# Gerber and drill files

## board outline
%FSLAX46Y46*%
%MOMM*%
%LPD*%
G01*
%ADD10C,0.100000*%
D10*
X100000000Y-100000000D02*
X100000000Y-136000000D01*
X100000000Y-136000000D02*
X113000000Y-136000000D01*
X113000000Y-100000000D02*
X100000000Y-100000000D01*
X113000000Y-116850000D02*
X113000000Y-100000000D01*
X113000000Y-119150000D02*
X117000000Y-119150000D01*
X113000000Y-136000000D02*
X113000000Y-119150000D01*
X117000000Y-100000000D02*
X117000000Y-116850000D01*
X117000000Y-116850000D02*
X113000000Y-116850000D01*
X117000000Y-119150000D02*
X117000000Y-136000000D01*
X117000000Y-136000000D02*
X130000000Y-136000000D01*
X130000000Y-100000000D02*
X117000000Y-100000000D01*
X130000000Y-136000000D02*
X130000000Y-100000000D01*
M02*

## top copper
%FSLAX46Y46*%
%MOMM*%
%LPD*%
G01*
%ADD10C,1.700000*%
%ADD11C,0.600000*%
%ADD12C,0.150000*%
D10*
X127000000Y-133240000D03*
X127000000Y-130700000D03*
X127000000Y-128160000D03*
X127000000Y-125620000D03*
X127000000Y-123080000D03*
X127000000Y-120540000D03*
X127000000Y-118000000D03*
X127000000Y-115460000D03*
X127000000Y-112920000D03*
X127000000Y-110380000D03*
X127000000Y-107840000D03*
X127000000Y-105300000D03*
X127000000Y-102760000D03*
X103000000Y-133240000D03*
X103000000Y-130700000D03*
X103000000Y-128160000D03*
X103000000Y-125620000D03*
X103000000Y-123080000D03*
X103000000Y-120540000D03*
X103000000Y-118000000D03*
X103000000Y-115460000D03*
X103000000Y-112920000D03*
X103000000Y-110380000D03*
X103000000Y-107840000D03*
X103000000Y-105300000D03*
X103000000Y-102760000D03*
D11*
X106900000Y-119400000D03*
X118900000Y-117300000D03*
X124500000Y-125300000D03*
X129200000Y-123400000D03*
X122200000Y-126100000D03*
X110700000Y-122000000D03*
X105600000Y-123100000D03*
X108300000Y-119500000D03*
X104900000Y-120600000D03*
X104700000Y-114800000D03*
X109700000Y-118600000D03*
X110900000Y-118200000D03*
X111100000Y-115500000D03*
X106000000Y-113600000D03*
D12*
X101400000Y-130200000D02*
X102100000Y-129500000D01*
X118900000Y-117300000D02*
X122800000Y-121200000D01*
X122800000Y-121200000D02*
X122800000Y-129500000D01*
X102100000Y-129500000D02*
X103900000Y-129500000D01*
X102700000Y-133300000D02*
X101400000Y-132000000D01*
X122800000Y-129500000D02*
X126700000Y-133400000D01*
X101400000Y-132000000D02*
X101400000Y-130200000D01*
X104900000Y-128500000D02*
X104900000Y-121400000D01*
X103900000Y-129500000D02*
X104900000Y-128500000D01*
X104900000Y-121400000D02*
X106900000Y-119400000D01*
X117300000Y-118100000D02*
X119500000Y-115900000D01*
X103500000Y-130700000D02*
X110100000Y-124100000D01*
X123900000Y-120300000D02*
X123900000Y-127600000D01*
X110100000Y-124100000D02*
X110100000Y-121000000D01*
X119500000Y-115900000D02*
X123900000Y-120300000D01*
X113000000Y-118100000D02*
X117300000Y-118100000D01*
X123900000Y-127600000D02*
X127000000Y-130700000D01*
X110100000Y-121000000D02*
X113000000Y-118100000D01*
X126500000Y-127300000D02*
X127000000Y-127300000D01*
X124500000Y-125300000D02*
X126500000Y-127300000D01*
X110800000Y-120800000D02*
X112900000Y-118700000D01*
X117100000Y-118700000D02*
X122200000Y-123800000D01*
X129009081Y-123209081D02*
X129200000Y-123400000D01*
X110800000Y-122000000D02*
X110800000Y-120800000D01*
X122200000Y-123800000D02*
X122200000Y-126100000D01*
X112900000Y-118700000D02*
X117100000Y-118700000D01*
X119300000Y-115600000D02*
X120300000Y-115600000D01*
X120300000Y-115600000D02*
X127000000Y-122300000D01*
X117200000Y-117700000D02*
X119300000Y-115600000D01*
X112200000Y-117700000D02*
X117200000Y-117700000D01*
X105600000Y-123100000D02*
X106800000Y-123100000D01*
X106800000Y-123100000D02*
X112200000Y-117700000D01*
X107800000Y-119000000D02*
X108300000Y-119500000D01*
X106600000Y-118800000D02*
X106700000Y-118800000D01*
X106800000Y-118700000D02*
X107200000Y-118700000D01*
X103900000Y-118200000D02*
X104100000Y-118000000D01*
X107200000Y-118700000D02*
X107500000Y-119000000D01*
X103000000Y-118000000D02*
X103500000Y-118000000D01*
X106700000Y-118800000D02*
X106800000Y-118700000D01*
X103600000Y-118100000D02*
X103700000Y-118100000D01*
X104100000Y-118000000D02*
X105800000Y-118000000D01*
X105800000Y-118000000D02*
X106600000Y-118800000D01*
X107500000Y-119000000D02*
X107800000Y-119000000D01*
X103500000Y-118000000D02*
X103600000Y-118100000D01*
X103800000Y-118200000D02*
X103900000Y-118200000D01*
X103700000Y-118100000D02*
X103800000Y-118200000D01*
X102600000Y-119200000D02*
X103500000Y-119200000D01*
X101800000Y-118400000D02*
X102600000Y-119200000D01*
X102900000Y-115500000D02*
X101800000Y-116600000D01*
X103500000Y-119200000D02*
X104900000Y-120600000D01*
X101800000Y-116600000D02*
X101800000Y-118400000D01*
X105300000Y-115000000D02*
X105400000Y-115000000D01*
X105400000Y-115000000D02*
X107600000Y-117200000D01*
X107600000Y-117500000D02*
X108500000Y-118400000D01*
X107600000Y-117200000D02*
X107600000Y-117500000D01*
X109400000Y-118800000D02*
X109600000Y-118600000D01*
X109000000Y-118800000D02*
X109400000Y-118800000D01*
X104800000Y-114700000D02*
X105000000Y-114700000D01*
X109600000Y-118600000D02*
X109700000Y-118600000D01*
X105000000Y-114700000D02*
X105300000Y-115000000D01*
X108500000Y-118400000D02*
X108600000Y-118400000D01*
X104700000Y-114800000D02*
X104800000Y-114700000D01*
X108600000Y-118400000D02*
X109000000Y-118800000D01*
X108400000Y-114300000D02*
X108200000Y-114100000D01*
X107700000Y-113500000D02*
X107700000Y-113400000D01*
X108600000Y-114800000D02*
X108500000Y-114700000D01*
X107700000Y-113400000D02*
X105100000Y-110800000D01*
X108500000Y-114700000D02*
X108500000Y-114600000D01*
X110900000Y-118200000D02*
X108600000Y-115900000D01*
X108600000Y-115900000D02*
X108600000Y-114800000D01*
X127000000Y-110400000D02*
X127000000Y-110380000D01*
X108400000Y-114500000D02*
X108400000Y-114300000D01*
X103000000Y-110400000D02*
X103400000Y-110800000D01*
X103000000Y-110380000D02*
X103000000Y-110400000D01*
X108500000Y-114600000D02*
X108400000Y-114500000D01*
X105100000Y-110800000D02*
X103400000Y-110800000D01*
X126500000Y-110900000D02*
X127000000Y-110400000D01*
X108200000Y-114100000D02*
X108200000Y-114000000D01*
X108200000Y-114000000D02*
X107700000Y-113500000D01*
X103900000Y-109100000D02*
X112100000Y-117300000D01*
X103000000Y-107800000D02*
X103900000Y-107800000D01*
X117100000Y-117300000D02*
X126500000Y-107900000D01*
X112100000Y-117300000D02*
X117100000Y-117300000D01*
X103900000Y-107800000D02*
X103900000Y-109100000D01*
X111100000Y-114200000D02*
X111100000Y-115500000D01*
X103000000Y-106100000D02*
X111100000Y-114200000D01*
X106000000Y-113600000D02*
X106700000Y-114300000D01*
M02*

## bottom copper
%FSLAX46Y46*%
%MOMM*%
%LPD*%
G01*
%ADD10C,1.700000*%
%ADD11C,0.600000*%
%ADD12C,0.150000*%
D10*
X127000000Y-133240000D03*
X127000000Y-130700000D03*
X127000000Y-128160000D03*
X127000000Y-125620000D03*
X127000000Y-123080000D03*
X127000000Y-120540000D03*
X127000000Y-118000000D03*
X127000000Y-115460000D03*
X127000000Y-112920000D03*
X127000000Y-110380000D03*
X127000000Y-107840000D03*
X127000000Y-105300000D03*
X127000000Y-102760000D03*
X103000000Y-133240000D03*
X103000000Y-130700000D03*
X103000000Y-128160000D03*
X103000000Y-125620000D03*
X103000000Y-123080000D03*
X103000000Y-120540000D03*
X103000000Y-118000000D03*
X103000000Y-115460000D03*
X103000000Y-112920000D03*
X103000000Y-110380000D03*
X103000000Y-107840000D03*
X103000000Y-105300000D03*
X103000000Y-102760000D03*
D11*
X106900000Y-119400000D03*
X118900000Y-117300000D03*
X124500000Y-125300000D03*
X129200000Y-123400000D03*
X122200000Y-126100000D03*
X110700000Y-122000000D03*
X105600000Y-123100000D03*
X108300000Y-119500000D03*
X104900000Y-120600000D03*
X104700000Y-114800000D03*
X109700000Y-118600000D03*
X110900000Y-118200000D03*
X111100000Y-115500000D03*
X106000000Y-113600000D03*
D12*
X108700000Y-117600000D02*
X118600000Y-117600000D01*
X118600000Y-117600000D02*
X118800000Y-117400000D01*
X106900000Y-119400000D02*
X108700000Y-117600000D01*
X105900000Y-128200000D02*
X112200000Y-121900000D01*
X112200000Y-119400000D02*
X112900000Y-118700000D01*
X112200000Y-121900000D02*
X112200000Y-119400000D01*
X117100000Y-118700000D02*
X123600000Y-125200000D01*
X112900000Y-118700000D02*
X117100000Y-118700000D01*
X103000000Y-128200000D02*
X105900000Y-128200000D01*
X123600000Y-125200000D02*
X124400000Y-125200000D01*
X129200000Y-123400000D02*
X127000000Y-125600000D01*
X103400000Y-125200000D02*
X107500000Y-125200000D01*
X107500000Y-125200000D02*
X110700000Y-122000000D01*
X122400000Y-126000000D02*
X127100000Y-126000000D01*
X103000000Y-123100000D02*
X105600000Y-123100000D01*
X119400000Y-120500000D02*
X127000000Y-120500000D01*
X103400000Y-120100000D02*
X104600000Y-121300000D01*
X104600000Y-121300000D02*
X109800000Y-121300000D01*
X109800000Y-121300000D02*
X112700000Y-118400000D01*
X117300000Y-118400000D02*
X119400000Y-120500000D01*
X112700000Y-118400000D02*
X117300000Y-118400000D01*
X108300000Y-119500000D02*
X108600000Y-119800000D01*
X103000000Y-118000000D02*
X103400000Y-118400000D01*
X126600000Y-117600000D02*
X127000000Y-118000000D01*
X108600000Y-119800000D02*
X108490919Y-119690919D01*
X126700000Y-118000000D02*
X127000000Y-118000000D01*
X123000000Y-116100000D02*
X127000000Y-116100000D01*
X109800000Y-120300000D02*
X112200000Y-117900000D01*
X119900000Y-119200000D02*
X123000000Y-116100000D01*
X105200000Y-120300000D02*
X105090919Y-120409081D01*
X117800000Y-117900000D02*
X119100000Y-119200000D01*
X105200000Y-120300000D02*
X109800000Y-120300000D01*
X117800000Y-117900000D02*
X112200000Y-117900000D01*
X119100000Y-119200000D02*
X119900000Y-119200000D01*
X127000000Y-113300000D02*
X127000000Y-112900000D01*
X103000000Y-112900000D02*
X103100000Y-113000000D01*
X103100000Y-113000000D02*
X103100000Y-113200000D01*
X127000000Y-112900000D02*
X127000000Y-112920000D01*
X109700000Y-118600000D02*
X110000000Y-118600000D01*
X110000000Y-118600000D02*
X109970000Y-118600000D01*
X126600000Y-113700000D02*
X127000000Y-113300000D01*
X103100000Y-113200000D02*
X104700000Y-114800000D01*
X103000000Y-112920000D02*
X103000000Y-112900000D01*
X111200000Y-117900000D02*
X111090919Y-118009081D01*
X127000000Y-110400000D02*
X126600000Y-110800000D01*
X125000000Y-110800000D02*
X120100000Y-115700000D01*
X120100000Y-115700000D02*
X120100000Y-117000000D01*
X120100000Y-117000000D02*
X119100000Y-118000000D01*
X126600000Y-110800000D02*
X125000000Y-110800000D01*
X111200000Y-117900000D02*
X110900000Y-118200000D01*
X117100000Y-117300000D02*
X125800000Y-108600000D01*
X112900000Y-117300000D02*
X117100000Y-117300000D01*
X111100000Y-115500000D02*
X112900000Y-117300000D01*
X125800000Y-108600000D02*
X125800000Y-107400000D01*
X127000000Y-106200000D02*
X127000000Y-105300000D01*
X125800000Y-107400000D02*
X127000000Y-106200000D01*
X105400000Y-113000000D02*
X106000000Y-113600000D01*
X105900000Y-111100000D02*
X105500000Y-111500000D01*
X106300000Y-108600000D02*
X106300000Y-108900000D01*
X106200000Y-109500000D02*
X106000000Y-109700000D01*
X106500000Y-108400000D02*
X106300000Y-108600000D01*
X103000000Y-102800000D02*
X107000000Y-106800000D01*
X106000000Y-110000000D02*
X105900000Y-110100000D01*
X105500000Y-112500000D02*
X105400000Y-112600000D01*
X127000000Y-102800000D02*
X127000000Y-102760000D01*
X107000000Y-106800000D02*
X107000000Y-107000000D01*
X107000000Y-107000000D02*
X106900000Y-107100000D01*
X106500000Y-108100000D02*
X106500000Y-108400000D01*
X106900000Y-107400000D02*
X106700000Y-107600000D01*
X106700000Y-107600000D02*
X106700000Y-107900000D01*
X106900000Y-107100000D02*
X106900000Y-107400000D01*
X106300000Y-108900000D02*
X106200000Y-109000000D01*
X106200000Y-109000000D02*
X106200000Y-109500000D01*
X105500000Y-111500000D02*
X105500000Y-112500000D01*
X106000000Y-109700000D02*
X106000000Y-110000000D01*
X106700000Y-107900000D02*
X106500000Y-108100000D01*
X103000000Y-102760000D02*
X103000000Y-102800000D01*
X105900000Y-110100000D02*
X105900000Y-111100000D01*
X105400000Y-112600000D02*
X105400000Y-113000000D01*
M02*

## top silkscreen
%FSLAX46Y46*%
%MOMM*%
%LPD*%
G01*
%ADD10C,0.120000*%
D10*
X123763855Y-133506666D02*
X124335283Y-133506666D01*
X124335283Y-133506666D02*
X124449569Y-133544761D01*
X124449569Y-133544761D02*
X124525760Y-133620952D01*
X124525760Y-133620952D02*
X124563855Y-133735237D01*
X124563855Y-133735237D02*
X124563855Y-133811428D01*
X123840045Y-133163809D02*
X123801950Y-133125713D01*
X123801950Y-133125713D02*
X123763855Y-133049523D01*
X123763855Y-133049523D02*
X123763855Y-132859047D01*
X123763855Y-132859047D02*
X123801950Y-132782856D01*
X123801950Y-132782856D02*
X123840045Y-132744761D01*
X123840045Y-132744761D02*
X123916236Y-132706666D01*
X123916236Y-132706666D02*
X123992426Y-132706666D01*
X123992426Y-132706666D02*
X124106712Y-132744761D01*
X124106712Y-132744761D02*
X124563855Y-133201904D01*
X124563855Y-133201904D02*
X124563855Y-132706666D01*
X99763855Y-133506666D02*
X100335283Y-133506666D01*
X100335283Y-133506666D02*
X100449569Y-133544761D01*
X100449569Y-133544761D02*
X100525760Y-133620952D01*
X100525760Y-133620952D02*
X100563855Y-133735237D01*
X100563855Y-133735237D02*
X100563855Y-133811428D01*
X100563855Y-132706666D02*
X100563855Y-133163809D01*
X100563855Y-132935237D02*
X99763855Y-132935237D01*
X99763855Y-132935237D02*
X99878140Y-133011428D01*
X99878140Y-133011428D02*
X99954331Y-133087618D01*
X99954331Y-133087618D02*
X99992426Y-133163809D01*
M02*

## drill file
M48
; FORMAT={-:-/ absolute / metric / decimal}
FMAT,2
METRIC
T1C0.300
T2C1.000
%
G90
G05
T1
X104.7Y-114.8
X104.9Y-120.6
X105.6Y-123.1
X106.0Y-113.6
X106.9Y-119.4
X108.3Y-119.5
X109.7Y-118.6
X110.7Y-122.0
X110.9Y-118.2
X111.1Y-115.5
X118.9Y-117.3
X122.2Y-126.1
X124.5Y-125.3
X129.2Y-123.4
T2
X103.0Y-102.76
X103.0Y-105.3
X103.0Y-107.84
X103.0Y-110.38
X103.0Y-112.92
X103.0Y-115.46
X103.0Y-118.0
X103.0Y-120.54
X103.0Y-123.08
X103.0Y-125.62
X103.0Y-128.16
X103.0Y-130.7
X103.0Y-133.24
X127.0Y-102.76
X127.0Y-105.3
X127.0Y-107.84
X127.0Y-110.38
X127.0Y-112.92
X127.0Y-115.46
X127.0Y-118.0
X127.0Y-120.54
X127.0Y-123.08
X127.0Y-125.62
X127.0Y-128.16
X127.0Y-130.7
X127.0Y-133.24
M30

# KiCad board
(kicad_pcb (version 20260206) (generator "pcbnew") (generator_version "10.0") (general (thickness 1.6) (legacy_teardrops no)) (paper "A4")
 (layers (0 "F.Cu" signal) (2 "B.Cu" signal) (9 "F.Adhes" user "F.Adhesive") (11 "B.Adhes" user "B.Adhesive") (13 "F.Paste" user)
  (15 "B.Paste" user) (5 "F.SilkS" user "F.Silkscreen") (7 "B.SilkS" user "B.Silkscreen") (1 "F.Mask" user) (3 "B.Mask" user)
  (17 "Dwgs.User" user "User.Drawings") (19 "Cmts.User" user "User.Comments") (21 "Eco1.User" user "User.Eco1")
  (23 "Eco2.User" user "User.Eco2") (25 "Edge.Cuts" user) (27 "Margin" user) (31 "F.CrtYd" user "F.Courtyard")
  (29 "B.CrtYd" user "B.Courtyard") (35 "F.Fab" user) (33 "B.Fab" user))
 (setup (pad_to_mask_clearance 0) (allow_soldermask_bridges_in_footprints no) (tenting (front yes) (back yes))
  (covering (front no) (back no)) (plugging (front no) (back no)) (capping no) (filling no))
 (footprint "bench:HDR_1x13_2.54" (layer "F.Cu") (at 127 133.24 90)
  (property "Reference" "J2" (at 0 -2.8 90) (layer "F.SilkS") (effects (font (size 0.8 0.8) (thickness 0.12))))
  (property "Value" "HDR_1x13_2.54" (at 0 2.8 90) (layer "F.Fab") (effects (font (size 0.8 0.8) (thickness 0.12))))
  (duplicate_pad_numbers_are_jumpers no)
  (pad "1" thru_hole circle (at 0 0 90) (size 1.7 1.7) (drill 1) (layers "*.Cu" "*.Mask") (remove_unused_layers no) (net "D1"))
  (pad "2" thru_hole circle (at 2.54 0 90) (size 1.7 1.7) (drill 1) (layers "*.Cu" "*.Mask") (remove_unused_layers no) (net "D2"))
  (pad "3" thru_hole circle (at 5.08 0 90) (size 1.7 1.7) (drill 1) (layers "*.Cu" "*.Mask") (remove_unused_layers no) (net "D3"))
  (pad "4" thru_hole circle (at 7.62 0 90) (size 1.7 1.7) (drill 1) (layers "*.Cu" "*.Mask") (remove_unused_layers no) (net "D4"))
  (pad "5" thru_hole circle (at 10.16 0 90) (size 1.7 1.7) (drill 1) (layers "*.Cu" "*.Mask") (remove_unused_layers no) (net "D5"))
  (pad "6" thru_hole circle (at 12.7 0 90) (size 1.7 1.7) (drill 1) (layers "*.Cu" "*.Mask") (remove_unused_layers no) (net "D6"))
  (pad "7" thru_hole circle (at 15.24 0 90) (size 1.7 1.7) (drill 1) (layers "*.Cu" "*.Mask") (remove_unused_layers no) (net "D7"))
  (pad "8" thru_hole circle (at 17.78 0 90) (size 1.7 1.7) (drill 1) (layers "*.Cu" "*.Mask") (remove_unused_layers no) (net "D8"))
  (pad "9" thru_hole circle (at 20.32 0 90) (size 1.7 1.7) (drill 1) (layers "*.Cu" "*.Mask") (remove_unused_layers no) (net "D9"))
  (pad "10" thru_hole circle (at 22.86 0 90) (size 1.7 1.7) (drill 1) (layers "*.Cu" "*.Mask") (remove_unused_layers no) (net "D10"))
  (pad "11" thru_hole circle (at 25.4 0 90) (size 1.7 1.7) (drill 1) (layers "*.Cu" "*.Mask") (remove_unused_layers no) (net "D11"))
  (pad "12" thru_hole circle (at 27.94 0 90) (size 1.7 1.7) (drill 1) (layers "*.Cu" "*.Mask") (remove_unused_layers no) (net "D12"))
  (pad "13" thru_hole circle (at 30.48 0 90) (size 1.7 1.7) (drill 1) (layers "*.Cu" "*.Mask") (remove_unused_layers no) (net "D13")))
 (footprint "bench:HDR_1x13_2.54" (layer "F.Cu") (at 103 133.24 90)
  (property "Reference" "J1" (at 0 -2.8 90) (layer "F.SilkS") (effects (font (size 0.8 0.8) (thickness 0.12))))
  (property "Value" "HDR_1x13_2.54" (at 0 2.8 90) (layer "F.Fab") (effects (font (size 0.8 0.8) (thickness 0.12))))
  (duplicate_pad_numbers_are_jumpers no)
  (pad "1" thru_hole circle (at 0 0 90) (size 1.7 1.7) (drill 1) (layers "*.Cu" "*.Mask") (remove_unused_layers no) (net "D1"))
  (pad "2" thru_hole circle (at 2.54 0 90) (size 1.7 1.7) (drill 1) (layers "*.Cu" "*.Mask") (remove_unused_layers no) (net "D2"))
  (pad "3" thru_hole circle (at 5.08 0 90) (size 1.7 1.7) (drill 1) (layers "*.Cu" "*.Mask") (remove_unused_layers no) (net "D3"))
  (pad "4" thru_hole circle (at 7.62 0 90) (size 1.7 1.7) (drill 1) (layers "*.Cu" "*.Mask") (remove_unused_layers no) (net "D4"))
  (pad "5" thru_hole circle (at 10.16 0 90) (size 1.7 1.7) (drill 1) (layers "*.Cu" "*.Mask") (remove_unused_layers no) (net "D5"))
  (pad "6" thru_hole circle (at 12.7 0 90) (size 1.7 1.7) (drill 1) (layers "*.Cu" "*.Mask") (remove_unused_layers no) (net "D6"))
  (pad "7" thru_hole circle (at 15.24 0 90) (size 1.7 1.7) (drill 1) (layers "*.Cu" "*.Mask") (remove_unused_layers no) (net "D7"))
  (pad "8" thru_hole circle (at 17.78 0 90) (size 1.7 1.7) (drill 1) (layers "*.Cu" "*.Mask") (remove_unused_layers no) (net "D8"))
  (pad "9" thru_hole circle (at 20.32 0 90) (size 1.7 1.7) (drill 1) (layers "*.Cu" "*.Mask") (remove_unused_layers no) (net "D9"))
  (pad "10" thru_hole circle (at 22.86 0 90) (size 1.7 1.7) (drill 1) (layers "*.Cu" "*.Mask") (remove_unused_layers no) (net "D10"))
  (pad "11" thru_hole circle (at 25.4 0 90) (size 1.7 1.7) (drill 1) (layers "*.Cu" "*.Mask") (remove_unused_layers no) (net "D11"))
  (pad "12" thru_hole circle (at 27.94 0 90) (size 1.7 1.7) (drill 1) (layers "*.Cu" "*.Mask") (remove_unused_layers no) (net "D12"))
  (pad "13" thru_hole circle (at 30.48 0 90) (size 1.7 1.7) (drill 1) (layers "*.Cu" "*.Mask") (remove_unused_layers no) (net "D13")))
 (gr_line (start 100 100) (end 100 136) (stroke (width 0.1) (type solid)) (layer "Edge.Cuts"))
 (gr_line (start 100 136) (end 113 136) (stroke (width 0.1) (type solid)) (layer "Edge.Cuts"))
 (gr_line (start 113 100) (end 100 100) (stroke (width 0.1) (type solid)) (layer "Edge.Cuts"))
 (gr_line (start 113 116.85) (end 113 100) (stroke (width 0.1) (type solid)) (layer "Edge.Cuts"))
 (gr_line (start 113 119.15) (end 117 119.15) (stroke (width 0.1) (type solid)) (layer "Edge.Cuts"))
 (gr_line (start 113 136) (end 113 119.15) (stroke (width 0.1) (type solid)) (layer "Edge.Cuts"))
 (gr_line (start 117 100) (end 117 116.85) (stroke (width 0.1) (type solid)) (layer "Edge.Cuts"))
 (gr_line (start 117 116.85) (end 113 116.85) (stroke (width 0.1) (type solid)) (layer "Edge.Cuts"))
 (gr_line (start 117 119.15) (end 117 136) (stroke (width 0.1) (type solid)) (layer "Edge.Cuts"))
 (gr_line (start 117 136) (end 130 136) (stroke (width 0.1) (type solid)) (layer "Edge.Cuts"))
 (gr_line (start 130 100) (end 117 100) (stroke (width 0.1) (type solid)) (layer "Edge.Cuts"))
 (gr_line (start 130 136) (end 130 100) (stroke (width 0.1) (type solid)) (layer "Edge.Cuts"))
 (segment (start 101.4 130.2) (end 102.1 129.5) (width 0.15) (layer "F.Cu") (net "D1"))
 (segment (start 118.9 117.3) (end 122.8 121.2) (width 0.15) (layer "F.Cu") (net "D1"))
 (segment (start 122.8 121.2) (end 122.8 129.5) (width 0.15) (layer "F.Cu") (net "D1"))
 (segment (start 102.1 129.5) (end 103.9 129.5) (width 0.15) (layer "F.Cu") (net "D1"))
 (segment (start 102.7 133.3) (end 101.4 132) (width 0.15) (layer "F.Cu") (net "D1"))
 (segment (start 122.8 129.5) (end 126.7 133.4) (width 0.15) (layer "F.Cu") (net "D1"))
 (segment (start 101.4 132) (end 101.4 130.2) (width 0.15) (layer "F.Cu") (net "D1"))
 (segment (start 104.9 128.5) (end 104.9 121.4) (width 0.15) (layer "F.Cu") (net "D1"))
 (segment (start 103.9 129.5) (end 104.9 128.5) (width 0.15) (layer "F.Cu") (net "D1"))
 (segment (start 104.9 121.4) (end 106.9 119.4) (width 0.15) (layer "F.Cu") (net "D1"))
 (via (at 106.9 119.4) (size 0.6) (drill 0.3) (layers "F.Cu" "B.Cu") (capping no) (covering (front no) (back no))
  (plugging (front no) (back no)) (filling no) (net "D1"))
 (via (at 118.9 117.3) (size 0.6) (drill 0.3) (layers "F.Cu" "B.Cu") (capping no) (covering (front no) (back no))
  (plugging (front no) (back no)) (filling no) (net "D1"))
 (segment (start 108.7 117.6) (end 118.6 117.6) (width 0.15) (layer "B.Cu") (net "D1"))
 (segment (start 118.6 117.6) (end 118.8 117.4) (width 0.15) (layer "B.Cu") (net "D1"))
 (segment (start 106.9 119.4) (end 108.7 117.6) (width 0.15) (layer "B.Cu") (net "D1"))
 (segment (start 117.3 118.1) (end 119.5 115.9) (width 0.15) (layer "F.Cu") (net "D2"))
 (segment (start 103.5 130.7) (end 110.1 124.1) (width 0.15) (layer "F.Cu") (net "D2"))
 (segment (start 123.9 120.3) (end 123.9 127.6) (width 0.15) (layer "F.Cu") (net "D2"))
 (segment (start 110.1 124.1) (end 110.1 121) (width 0.15) (layer "F.Cu") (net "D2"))
 (segment (start 119.5 115.9) (end 123.9 120.3) (width 0.15) (layer "F.Cu") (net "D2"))
 (segment (start 113 118.1) (end 117.3 118.1) (width 0.15) (layer "F.Cu") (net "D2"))
 (segment (start 123.9 127.6) (end 127 130.7) (width 0.15) (layer "F.Cu") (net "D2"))
 (segment (start 110.1 121) (end 113 118.1) (width 0.15) (layer "F.Cu") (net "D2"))
 (segment (start 126.5 127.3) (end 127 127.3) (width 0.15) (layer "F.Cu") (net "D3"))
 (segment (start 124.5 125.3) (end 126.5 127.3) (width 0.15) (layer "F.Cu") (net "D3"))
 (via (at 124.5 125.3) (size 0.6) (drill 0.3) (layers "F.Cu" "B.Cu") (capping no) (covering (front no) (back no))
  (plugging (front no) (back no)) (filling no) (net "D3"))
 (segment (start 105.9 128.2) (end 112.2 121.9) (width 0.15) (layer "B.Cu") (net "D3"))
 (segment (start 112.2 119.4) (end 112.9 118.7) (width 0.15) (layer "B.Cu") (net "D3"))
 (segment (start 112.2 121.9) (end 112.2 119.4) (width 0.15) (layer "B.Cu") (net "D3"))
 (segment (start 117.1 118.7) (end 123.6 125.2) (width 0.15) (layer "B.Cu") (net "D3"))
 (segment (start 112.9 118.7) (end 117.1 118.7) (width 0.15) (layer "B.Cu") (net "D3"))
 (segment (start 103 128.2) (end 105.9 128.2) (width 0.15) (layer "B.Cu") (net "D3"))
 (segment (start 123.6 125.2) (end 124.4 125.2) (width 0.15) (layer "B.Cu") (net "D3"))
 (segment (start 110.8 120.8) (end 112.9 118.7) (width 0.15) (layer "F.Cu") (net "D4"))
 (segment (start 117.1 118.7) (end 122.2 123.8) (width 0.15) (layer "F.Cu") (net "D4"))
 (segment (start 129.009081 123.209081) (end 129.2 123.4) (width 0.15) (layer "F.Cu") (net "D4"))
 (segment (start 110.8 122) (end 110.8 120.8) (width 0.15) (layer "F.Cu") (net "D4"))
 (segment (start 122.2 123.8) (end 122.2 126.1) (width 0.15) (layer "F.Cu") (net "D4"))
 (segment (start 112.9 118.7) (end 117.1 118.7) (width 0.15) (layer "F.Cu") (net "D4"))
 (via (at 129.2 123.4) (size 0.6) (drill 0.3) (layers "F.Cu" "B.Cu") (capping no) (covering (front no) (back no))
  (plugging (front no) (back no)) (filling no) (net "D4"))
 (via (at 122.2 126.1) (size 0.6) (drill 0.3) (layers "F.Cu" "B.Cu") (capping no) (covering (front no) (back no))
  (plugging (front no) (back no)) (filling no) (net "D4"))
 (via (at 110.7 122) (size 0.6) (drill 0.3) (layers "F.Cu" "B.Cu") (capping no) (covering (front no) (back no))
  (plugging (front no) (back no)) (filling no) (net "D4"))
 (segment (start 129.2 123.4) (end 127 125.6) (width 0.15) (layer "B.Cu") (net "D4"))
 (segment (start 103.4 125.2) (end 107.5 125.2) (width 0.15) (layer "B.Cu") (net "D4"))
 (segment (start 107.5 125.2) (end 110.7 122) (width 0.15) (layer "B.Cu") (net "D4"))
 (segment (start 122.4 126) (end 127.1 126) (width 0.15) (layer "B.Cu") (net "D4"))
 (segment (start 119.3 115.6) (end 120.3 115.6) (width 0.15) (layer "F.Cu") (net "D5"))
 (segment (start 120.3 115.6) (end 127 122.3) (width 0.15) (layer "F.Cu") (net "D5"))
 (segment (start 117.2 117.7) (end 119.3 115.6) (width 0.15) (layer "F.Cu") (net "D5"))
 (segment (start 112.2 117.7) (end 117.2 117.7) (width 0.15) (layer "F.Cu") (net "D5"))
 (segment (start 105.6 123.1) (end 106.8 123.1) (width 0.15) (layer "F.Cu") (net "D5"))
 (segment (start 106.8 123.1) (end 112.2 117.7) (width 0.15) (layer "F.Cu") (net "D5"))
 (via (at 105.6 123.1) (size 0.6) (drill 0.3) (layers "F.Cu" "B.Cu") (capping no) (covering (front no) (back no))
  (plugging (front no) (back no)) (filling no) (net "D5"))
 (segment (start 103 123.1) (end 105.6 123.1) (width 0.15) (layer "B.Cu") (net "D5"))
 (segment (start 119.4 120.5) (end 127 120.5) (width 0.15) (layer "B.Cu") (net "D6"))
 (segment (start 103.4 120.1) (end 104.6 121.3) (width 0.15) (layer "B.Cu") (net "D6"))
 (segment (start 104.6 121.3) (end 109.8 121.3) (width 0.15) (layer "B.Cu") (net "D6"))
 (segment (start 109.8 121.3) (end 112.7 118.4) (width 0.15) (layer "B.Cu") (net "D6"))
 (segment (start 117.3 118.4) (end 119.4 120.5) (width 0.15) (layer "B.Cu") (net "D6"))
 (segment (start 112.7 118.4) (end 117.3 118.4) (width 0.15) (layer "B.Cu") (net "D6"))
 (segment (start 107.8 119) (end 108.3 119.5) (width 0.15) (layer "F.Cu") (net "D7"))
 (segment (start 106.6 118.8) (end 106.7 118.8) (width 0.15) (layer "F.Cu") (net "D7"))
 (segment (start 106.8 118.7) (end 107.2 118.7) (width 0.15) (layer "F.Cu") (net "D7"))
 (segment (start 103.9 118.2) (end 104.1 118) (width 0.15) (layer "F.Cu") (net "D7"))
 (segment (start 107.2 118.7) (end 107.5 119) (width 0.15) (layer "F.Cu") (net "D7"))
 (segment (start 103 118) (end 103.5 118) (width 0.15) (layer "F.Cu") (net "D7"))
 (segment (start 106.7 118.8) (end 106.8 118.7) (width 0.15) (layer "F.Cu") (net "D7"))
 (segment (start 103.6 118.1) (end 103.7 118.1) (width 0.15) (layer "F.Cu") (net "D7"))
 (segment (start 104.1 118) (end 105.8 118) (width 0.15) (layer "F.Cu") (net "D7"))
 (segment (start 105.8 118) (end 106.6 118.8) (width 0.15) (layer "F.Cu") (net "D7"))
 (segment (start 107.5 119) (end 107.8 119) (width 0.15) (layer "F.Cu") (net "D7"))
 (segment (start 103.5 118) (end 103.6 118.1) (width 0.15) (layer "F.Cu") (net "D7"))
 (segment (start 103.8 118.2) (end 103.9 118.2) (width 0.15) (layer "F.Cu") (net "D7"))
 (segment (start 103.7 118.1) (end 103.8 118.2) (width 0.15) (layer "F.Cu") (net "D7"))
 (via (at 108.3 119.5) (size 0.6) (drill 0.3) (layers "F.Cu" "B.Cu") (capping no) (covering (front no) (back no))
  (plugging (front no) (back no)) (filling no) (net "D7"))
 (segment (start 108.3 119.5) (end 108.6 119.8) (width 0.15) (layer "B.Cu") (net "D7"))
 (segment (start 103 118) (end 103.4 118.4) (width 0.15) (layer "B.Cu") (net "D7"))
 (segment (start 126.6 117.6) (end 127 118) (width 0.15) (layer "B.Cu") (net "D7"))
 (segment (start 108.6 119.8) (end 108.490919 119.690919) (width 0.15) (layer "B.Cu") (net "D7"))
 (segment (start 126.7 118) (end 127 118) (width 0.15) (layer "B.Cu") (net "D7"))
 (segment (start 102.6 119.2) (end 103.5 119.2) (width 0.15) (layer "F.Cu") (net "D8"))
 (segment (start 101.8 118.4) (end 102.6 119.2) (width 0.15) (layer "F.Cu") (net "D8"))
 (segment (start 102.9 115.5) (end 101.8 116.6) (width 0.15) (layer "F.Cu") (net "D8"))
 (segment (start 103.5 119.2) (end 104.9 120.6) (width 0.15) (layer "F.Cu") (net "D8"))
 (segment (start 101.8 116.6) (end 101.8 118.4) (width 0.15) (layer "F.Cu") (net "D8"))
 (via (at 104.9 120.6) (size 0.6) (drill 0.3) (layers "F.Cu" "B.Cu") (capping no) (covering (front no) (back no))
  (plugging (front no) (back no)) (filling no) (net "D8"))
 (segment (start 123 116.1) (end 127 116.1) (width 0.15) (layer "B.Cu") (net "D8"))
 (segment (start 109.8 120.3) (end 112.2 117.9) (width 0.15) (layer "B.Cu") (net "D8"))
 (segment (start 119.9 119.2) (end 123 116.1) (width 0.15) (layer "B.Cu") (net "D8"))
 (segment (start 105.2 120.3) (end 105.090919 120.409081) (width 0.15) (layer "B.Cu") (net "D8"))
 (segment (start 117.8 117.9) (end 119.1 119.2) (width 0.15) (layer "B.Cu") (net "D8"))
 (segment (start 105.2 120.3) (end 109.8 120.3) (width 0.15) (layer "B.Cu") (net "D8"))
 (segment (start 117.8 117.9) (end 112.2 117.9) (width 0.15) (layer "B.Cu") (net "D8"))
 (segment (start 119.1 119.2) (end 119.9 119.2) (width 0.15) (layer "B.Cu") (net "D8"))
 (segment (start 105.3 115) (end 105.4 115) (width 0.15) (layer "F.Cu") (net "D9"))
 (segment (start 105.4 115) (end 107.6 117.2) (width 0.15) (layer "F.Cu") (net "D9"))
 (segment (start 107.6 117.5) (end 108.5 118.4) (width 0.15) (layer "F.Cu") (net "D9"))
 (segment (start 107.6 117.2) (end 107.6 117.5) (width 0.15) (layer "F.Cu") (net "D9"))
 (segment (start 109.4 118.8) (end 109.6 118.6) (width 0.15) (layer "F.Cu") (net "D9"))
 (segment (start 109 118.8) (end 109.4 118.8) (width 0.15) (layer "F.Cu") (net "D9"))
 (segment (start 104.8 114.7) (end 105 114.7) (width 0.15) (layer "F.Cu") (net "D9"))
 (segment (start 109.6 118.6) (end 109.7 118.6) (width 0.15) (layer "F.Cu") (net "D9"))
 (segment (start 105 114.7) (end 105.3 115) (width 0.15) (layer "F.Cu") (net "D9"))
 (segment (start 108.5 118.4) (end 108.6 118.4) (width 0.15) (layer "F.Cu") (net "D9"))
 (segment (start 104.7 114.8) (end 104.8 114.7) (width 0.15) (layer "F.Cu") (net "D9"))
 (segment (start 108.6 118.4) (end 109 118.8) (width 0.15) (layer "F.Cu") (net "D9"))
 (via (at 104.7 114.8) (size 0.6) (drill 0.3) (layers "F.Cu" "B.Cu") (capping no) (covering (front no) (back no))
  (plugging (front no) (back no)) (filling no) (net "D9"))
 (via (at 109.7 118.6) (size 0.6) (drill 0.3) (layers "F.Cu" "B.Cu") (capping no) (covering (front no) (back no))
  (plugging (front no) (back no)) (filling no) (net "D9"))
 (segment (start 127 113.3) (end 127 112.9) (width 0.15) (layer "B.Cu") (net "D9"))
 (segment (start 103 112.9) (end 103.1 113) (width 0.15) (layer "B.Cu") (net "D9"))
 (segment (start 103.1 113) (end 103.1 113.2) (width 0.15) (layer "B.Cu") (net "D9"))
 (segment (start 127 112.9) (end 127 112.92) (width 0.15) (layer "B.Cu") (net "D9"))
 (segment (start 109.7 118.6) (end 110 118.6) (width 0.15) (layer "B.Cu") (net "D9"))
 (segment (start 110 118.6) (end 109.97 118.6) (width 0.15) (layer "B.Cu") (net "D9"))
 (segment (start 126.6 113.7) (end 127 113.3) (width 0.15) (layer "B.Cu") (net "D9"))
 (segment (start 103.1 113.2) (end 104.7 114.8) (width 0.15) (layer "B.Cu") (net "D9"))
 (segment (start 103 112.92) (end 103 112.9) (width 0.15) (layer "B.Cu") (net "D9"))
 (segment (start 108.4 114.3) (end 108.2 114.1) (width 0.15) (layer "F.Cu") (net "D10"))
 (segment (start 107.7 113.5) (end 107.7 113.4) (width 0.15) (layer "F.Cu") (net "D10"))
 (segment (start 108.6 114.8) (end 108.5 114.7) (width 0.15) (layer "F.Cu") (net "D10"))
 (segment (start 107.7 113.4) (end 105.1 110.8) (width 0.15) (layer "F.Cu") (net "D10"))
 (segment (start 108.5 114.7) (end 108.5 114.6) (width 0.15) (layer "F.Cu") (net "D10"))
 (segment (start 110.9 118.2) (end 108.6 115.9) (width 0.15) (layer "F.Cu") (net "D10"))
 (segment (start 108.6 115.9) (end 108.6 114.8) (width 0.15) (layer "F.Cu") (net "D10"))
 (segment (start 127 110.4) (end 127 110.38) (width 0.15) (layer "F.Cu") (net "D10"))
 (segment (start 108.4 114.5) (end 108.4 114.3) (width 0.15) (layer "F.Cu") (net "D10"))
 (segment (start 103 110.4) (end 103.4 110.8) (width 0.15) (layer "F.Cu") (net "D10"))
 (segment (start 103 110.38) (end 103 110.4) (width 0.15) (layer "F.Cu") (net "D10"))
 (segment (start 108.5 114.6) (end 108.4 114.5) (width 0.15) (layer "F.Cu") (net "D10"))
 (segment (start 105.1 110.8) (end 103.4 110.8) (width 0.15) (layer "F.Cu") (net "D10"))
 (segment (start 126.5 110.9) (end 127 110.4) (width 0.15) (layer "F.Cu") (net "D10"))
 (segment (start 108.2 114.1) (end 108.2 114) (width 0.15) (layer "F.Cu") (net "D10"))
 (segment (start 108.2 114) (end 107.7 113.5) (width 0.15) (layer "F.Cu") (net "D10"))
 (via (at 110.9 118.2) (size 0.6) (drill 0.3) (layers "F.Cu" "B.Cu") (capping no) (covering (front no) (back no))
  (plugging (front no) (back no)) (filling no) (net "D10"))
 (segment (start 111.2 117.9) (end 111.090919 118.009081) (width 0.15) (layer "B.Cu") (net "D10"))
 (segment (start 127 110.4) (end 126.6 110.8) (width 0.15) (layer "B.Cu") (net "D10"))
 (segment (start 125 110.8) (end 120.1 115.7) (width 0.15) (layer "B.Cu") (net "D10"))
 (segment (start 120.1 115.7) (end 120.1 117) (width 0.15) (layer "B.Cu") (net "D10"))
 (segment (start 120.1 117) (end 119.1 118) (width 0.15) (layer "B.Cu") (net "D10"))
 (segment (start 126.6 110.8) (end 125 110.8) (width 0.15) (layer "B.Cu") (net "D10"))
 (segment (start 111.2 117.9) (end 110.9 118.2) (width 0.15) (layer "B.Cu") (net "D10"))
 (segment (start 103.9 109.1) (end 112.1 117.3) (width 0.15) (layer "F.Cu") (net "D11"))
 (segment (start 103 107.8) (end 103.9 107.8) (width 0.15) (layer "F.Cu") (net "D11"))
 (segment (start 117.1 117.3) (end 126.5 107.9) (width 0.15) (layer "F.Cu") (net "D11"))
 (segment (start 112.1 117.3) (end 117.1 117.3) (width 0.15) (layer "F.Cu") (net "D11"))
 (segment (start 103.9 107.8) (end 103.9 109.1) (width 0.15) (layer "F.Cu") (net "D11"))
 (segment (start 111.1 114.2) (end 111.1 115.5) (width 0.15) (layer "F.Cu") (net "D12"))
 (segment (start 103 106.1) (end 111.1 114.2) (width 0.15) (layer "F.Cu") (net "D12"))
 (via (at 111.1 115.5) (size 0.6) (drill 0.3) (layers "F.Cu" "B.Cu") (capping no) (covering (front no) (back no))
  (plugging (front no) (back no)) (filling no) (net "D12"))
 (segment (start 117.1 117.3) (end 125.8 108.6) (width 0.15) (layer "B.Cu") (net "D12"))
 (segment (start 112.9 117.3) (end 117.1 117.3) (width 0.15) (layer "B.Cu") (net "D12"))
 (segment (start 111.1 115.5) (end 112.9 117.3) (width 0.15) (layer "B.Cu") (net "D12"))
 (segment (start 125.8 108.6) (end 125.8 107.4) (width 0.15) (layer "B.Cu") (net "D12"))
 (segment (start 127 106.2) (end 127 105.3) (width 0.15) (layer "B.Cu") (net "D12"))
 (segment (start 125.8 107.4) (end 127 106.2) (width 0.15) (layer "B.Cu") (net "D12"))
 (segment (start 106 113.6) (end 106.7 114.3) (width 0.15) (layer "F.Cu") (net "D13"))
 (via (at 106 113.6) (size 0.6) (drill 0.3) (layers "F.Cu" "B.Cu") (capping no) (covering (front no) (back no))
  (plugging (front no) (back no)) (filling no) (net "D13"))
 (segment (start 105.4 113) (end 106 113.6) (width 0.15) (layer "B.Cu") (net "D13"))
 (segment (start 105.9 111.1) (end 105.5 111.5) (width 0.15) (layer "B.Cu") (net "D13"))
 (segment (start 106.3 108.6) (end 106.3 108.9) (width 0.15) (layer "B.Cu") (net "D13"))
 (segment (start 106.2 109.5) (end 106 109.7) (width 0.15) (layer "B.Cu") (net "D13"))
 (segment (start 106.5 108.4) (end 106.3 108.6) (width 0.15) (layer "B.Cu") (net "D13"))
 (segment (start 103 102.8) (end 107 106.8) (width 0.15) (layer "B.Cu") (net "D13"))
 (segment (start 106 110) (end 105.9 110.1) (width 0.15) (layer "B.Cu") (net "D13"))
 (segment (start 105.5 112.5) (end 105.4 112.6) (width 0.15) (layer "B.Cu") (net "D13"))
 (segment (start 127 102.8) (end 127 102.76) (width 0.15) (layer "B.Cu") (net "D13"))
 (segment (start 107 106.8) (end 107 107) (width 0.15) (layer "B.Cu") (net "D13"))
 (segment (start 107 107) (end 106.9 107.1) (width 0.15) (layer "B.Cu") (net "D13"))
 (segment (start 106.5 108.1) (end 106.5 108.4) (width 0.15) (layer "B.Cu") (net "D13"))
 (segment (start 106.9 107.4) (end 106.7 107.6) (width 0.15) (layer "B.Cu") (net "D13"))
 (segment (start 106.7 107.6) (end 106.7 107.9) (width 0.15) (layer "B.Cu") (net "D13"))
 (segment (start 106.9 107.1) (end 106.9 107.4) (width 0.15) (layer "B.Cu") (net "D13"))
 (segment (start 106.3 108.9) (end 106.2 109) (width 0.15) (layer "B.Cu") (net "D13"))
 (segment (start 106.2 109) (end 106.2 109.5) (width 0.15) (layer "B.Cu") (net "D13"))
 (segment (start 105.5 111.5) (end 105.5 112.5) (width 0.15) (layer "B.Cu") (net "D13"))
 (segment (start 106 109.7) (end 106 110) (width 0.15) (layer "B.Cu") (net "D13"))
 (segment (start 106.7 107.9) (end 106.5 108.1) (width 0.15) (layer "B.Cu") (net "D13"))
 (segment (start 103 102.76) (end 103 102.8) (width 0.15) (layer "B.Cu") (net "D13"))
 (segment (start 105.9 110.1) (end 105.9 111.1) (width 0.15) (layer "B.Cu") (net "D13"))
 (segment (start 105.4 112.6) (end 105.4 113) (width 0.15) (layer "B.Cu") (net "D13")))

